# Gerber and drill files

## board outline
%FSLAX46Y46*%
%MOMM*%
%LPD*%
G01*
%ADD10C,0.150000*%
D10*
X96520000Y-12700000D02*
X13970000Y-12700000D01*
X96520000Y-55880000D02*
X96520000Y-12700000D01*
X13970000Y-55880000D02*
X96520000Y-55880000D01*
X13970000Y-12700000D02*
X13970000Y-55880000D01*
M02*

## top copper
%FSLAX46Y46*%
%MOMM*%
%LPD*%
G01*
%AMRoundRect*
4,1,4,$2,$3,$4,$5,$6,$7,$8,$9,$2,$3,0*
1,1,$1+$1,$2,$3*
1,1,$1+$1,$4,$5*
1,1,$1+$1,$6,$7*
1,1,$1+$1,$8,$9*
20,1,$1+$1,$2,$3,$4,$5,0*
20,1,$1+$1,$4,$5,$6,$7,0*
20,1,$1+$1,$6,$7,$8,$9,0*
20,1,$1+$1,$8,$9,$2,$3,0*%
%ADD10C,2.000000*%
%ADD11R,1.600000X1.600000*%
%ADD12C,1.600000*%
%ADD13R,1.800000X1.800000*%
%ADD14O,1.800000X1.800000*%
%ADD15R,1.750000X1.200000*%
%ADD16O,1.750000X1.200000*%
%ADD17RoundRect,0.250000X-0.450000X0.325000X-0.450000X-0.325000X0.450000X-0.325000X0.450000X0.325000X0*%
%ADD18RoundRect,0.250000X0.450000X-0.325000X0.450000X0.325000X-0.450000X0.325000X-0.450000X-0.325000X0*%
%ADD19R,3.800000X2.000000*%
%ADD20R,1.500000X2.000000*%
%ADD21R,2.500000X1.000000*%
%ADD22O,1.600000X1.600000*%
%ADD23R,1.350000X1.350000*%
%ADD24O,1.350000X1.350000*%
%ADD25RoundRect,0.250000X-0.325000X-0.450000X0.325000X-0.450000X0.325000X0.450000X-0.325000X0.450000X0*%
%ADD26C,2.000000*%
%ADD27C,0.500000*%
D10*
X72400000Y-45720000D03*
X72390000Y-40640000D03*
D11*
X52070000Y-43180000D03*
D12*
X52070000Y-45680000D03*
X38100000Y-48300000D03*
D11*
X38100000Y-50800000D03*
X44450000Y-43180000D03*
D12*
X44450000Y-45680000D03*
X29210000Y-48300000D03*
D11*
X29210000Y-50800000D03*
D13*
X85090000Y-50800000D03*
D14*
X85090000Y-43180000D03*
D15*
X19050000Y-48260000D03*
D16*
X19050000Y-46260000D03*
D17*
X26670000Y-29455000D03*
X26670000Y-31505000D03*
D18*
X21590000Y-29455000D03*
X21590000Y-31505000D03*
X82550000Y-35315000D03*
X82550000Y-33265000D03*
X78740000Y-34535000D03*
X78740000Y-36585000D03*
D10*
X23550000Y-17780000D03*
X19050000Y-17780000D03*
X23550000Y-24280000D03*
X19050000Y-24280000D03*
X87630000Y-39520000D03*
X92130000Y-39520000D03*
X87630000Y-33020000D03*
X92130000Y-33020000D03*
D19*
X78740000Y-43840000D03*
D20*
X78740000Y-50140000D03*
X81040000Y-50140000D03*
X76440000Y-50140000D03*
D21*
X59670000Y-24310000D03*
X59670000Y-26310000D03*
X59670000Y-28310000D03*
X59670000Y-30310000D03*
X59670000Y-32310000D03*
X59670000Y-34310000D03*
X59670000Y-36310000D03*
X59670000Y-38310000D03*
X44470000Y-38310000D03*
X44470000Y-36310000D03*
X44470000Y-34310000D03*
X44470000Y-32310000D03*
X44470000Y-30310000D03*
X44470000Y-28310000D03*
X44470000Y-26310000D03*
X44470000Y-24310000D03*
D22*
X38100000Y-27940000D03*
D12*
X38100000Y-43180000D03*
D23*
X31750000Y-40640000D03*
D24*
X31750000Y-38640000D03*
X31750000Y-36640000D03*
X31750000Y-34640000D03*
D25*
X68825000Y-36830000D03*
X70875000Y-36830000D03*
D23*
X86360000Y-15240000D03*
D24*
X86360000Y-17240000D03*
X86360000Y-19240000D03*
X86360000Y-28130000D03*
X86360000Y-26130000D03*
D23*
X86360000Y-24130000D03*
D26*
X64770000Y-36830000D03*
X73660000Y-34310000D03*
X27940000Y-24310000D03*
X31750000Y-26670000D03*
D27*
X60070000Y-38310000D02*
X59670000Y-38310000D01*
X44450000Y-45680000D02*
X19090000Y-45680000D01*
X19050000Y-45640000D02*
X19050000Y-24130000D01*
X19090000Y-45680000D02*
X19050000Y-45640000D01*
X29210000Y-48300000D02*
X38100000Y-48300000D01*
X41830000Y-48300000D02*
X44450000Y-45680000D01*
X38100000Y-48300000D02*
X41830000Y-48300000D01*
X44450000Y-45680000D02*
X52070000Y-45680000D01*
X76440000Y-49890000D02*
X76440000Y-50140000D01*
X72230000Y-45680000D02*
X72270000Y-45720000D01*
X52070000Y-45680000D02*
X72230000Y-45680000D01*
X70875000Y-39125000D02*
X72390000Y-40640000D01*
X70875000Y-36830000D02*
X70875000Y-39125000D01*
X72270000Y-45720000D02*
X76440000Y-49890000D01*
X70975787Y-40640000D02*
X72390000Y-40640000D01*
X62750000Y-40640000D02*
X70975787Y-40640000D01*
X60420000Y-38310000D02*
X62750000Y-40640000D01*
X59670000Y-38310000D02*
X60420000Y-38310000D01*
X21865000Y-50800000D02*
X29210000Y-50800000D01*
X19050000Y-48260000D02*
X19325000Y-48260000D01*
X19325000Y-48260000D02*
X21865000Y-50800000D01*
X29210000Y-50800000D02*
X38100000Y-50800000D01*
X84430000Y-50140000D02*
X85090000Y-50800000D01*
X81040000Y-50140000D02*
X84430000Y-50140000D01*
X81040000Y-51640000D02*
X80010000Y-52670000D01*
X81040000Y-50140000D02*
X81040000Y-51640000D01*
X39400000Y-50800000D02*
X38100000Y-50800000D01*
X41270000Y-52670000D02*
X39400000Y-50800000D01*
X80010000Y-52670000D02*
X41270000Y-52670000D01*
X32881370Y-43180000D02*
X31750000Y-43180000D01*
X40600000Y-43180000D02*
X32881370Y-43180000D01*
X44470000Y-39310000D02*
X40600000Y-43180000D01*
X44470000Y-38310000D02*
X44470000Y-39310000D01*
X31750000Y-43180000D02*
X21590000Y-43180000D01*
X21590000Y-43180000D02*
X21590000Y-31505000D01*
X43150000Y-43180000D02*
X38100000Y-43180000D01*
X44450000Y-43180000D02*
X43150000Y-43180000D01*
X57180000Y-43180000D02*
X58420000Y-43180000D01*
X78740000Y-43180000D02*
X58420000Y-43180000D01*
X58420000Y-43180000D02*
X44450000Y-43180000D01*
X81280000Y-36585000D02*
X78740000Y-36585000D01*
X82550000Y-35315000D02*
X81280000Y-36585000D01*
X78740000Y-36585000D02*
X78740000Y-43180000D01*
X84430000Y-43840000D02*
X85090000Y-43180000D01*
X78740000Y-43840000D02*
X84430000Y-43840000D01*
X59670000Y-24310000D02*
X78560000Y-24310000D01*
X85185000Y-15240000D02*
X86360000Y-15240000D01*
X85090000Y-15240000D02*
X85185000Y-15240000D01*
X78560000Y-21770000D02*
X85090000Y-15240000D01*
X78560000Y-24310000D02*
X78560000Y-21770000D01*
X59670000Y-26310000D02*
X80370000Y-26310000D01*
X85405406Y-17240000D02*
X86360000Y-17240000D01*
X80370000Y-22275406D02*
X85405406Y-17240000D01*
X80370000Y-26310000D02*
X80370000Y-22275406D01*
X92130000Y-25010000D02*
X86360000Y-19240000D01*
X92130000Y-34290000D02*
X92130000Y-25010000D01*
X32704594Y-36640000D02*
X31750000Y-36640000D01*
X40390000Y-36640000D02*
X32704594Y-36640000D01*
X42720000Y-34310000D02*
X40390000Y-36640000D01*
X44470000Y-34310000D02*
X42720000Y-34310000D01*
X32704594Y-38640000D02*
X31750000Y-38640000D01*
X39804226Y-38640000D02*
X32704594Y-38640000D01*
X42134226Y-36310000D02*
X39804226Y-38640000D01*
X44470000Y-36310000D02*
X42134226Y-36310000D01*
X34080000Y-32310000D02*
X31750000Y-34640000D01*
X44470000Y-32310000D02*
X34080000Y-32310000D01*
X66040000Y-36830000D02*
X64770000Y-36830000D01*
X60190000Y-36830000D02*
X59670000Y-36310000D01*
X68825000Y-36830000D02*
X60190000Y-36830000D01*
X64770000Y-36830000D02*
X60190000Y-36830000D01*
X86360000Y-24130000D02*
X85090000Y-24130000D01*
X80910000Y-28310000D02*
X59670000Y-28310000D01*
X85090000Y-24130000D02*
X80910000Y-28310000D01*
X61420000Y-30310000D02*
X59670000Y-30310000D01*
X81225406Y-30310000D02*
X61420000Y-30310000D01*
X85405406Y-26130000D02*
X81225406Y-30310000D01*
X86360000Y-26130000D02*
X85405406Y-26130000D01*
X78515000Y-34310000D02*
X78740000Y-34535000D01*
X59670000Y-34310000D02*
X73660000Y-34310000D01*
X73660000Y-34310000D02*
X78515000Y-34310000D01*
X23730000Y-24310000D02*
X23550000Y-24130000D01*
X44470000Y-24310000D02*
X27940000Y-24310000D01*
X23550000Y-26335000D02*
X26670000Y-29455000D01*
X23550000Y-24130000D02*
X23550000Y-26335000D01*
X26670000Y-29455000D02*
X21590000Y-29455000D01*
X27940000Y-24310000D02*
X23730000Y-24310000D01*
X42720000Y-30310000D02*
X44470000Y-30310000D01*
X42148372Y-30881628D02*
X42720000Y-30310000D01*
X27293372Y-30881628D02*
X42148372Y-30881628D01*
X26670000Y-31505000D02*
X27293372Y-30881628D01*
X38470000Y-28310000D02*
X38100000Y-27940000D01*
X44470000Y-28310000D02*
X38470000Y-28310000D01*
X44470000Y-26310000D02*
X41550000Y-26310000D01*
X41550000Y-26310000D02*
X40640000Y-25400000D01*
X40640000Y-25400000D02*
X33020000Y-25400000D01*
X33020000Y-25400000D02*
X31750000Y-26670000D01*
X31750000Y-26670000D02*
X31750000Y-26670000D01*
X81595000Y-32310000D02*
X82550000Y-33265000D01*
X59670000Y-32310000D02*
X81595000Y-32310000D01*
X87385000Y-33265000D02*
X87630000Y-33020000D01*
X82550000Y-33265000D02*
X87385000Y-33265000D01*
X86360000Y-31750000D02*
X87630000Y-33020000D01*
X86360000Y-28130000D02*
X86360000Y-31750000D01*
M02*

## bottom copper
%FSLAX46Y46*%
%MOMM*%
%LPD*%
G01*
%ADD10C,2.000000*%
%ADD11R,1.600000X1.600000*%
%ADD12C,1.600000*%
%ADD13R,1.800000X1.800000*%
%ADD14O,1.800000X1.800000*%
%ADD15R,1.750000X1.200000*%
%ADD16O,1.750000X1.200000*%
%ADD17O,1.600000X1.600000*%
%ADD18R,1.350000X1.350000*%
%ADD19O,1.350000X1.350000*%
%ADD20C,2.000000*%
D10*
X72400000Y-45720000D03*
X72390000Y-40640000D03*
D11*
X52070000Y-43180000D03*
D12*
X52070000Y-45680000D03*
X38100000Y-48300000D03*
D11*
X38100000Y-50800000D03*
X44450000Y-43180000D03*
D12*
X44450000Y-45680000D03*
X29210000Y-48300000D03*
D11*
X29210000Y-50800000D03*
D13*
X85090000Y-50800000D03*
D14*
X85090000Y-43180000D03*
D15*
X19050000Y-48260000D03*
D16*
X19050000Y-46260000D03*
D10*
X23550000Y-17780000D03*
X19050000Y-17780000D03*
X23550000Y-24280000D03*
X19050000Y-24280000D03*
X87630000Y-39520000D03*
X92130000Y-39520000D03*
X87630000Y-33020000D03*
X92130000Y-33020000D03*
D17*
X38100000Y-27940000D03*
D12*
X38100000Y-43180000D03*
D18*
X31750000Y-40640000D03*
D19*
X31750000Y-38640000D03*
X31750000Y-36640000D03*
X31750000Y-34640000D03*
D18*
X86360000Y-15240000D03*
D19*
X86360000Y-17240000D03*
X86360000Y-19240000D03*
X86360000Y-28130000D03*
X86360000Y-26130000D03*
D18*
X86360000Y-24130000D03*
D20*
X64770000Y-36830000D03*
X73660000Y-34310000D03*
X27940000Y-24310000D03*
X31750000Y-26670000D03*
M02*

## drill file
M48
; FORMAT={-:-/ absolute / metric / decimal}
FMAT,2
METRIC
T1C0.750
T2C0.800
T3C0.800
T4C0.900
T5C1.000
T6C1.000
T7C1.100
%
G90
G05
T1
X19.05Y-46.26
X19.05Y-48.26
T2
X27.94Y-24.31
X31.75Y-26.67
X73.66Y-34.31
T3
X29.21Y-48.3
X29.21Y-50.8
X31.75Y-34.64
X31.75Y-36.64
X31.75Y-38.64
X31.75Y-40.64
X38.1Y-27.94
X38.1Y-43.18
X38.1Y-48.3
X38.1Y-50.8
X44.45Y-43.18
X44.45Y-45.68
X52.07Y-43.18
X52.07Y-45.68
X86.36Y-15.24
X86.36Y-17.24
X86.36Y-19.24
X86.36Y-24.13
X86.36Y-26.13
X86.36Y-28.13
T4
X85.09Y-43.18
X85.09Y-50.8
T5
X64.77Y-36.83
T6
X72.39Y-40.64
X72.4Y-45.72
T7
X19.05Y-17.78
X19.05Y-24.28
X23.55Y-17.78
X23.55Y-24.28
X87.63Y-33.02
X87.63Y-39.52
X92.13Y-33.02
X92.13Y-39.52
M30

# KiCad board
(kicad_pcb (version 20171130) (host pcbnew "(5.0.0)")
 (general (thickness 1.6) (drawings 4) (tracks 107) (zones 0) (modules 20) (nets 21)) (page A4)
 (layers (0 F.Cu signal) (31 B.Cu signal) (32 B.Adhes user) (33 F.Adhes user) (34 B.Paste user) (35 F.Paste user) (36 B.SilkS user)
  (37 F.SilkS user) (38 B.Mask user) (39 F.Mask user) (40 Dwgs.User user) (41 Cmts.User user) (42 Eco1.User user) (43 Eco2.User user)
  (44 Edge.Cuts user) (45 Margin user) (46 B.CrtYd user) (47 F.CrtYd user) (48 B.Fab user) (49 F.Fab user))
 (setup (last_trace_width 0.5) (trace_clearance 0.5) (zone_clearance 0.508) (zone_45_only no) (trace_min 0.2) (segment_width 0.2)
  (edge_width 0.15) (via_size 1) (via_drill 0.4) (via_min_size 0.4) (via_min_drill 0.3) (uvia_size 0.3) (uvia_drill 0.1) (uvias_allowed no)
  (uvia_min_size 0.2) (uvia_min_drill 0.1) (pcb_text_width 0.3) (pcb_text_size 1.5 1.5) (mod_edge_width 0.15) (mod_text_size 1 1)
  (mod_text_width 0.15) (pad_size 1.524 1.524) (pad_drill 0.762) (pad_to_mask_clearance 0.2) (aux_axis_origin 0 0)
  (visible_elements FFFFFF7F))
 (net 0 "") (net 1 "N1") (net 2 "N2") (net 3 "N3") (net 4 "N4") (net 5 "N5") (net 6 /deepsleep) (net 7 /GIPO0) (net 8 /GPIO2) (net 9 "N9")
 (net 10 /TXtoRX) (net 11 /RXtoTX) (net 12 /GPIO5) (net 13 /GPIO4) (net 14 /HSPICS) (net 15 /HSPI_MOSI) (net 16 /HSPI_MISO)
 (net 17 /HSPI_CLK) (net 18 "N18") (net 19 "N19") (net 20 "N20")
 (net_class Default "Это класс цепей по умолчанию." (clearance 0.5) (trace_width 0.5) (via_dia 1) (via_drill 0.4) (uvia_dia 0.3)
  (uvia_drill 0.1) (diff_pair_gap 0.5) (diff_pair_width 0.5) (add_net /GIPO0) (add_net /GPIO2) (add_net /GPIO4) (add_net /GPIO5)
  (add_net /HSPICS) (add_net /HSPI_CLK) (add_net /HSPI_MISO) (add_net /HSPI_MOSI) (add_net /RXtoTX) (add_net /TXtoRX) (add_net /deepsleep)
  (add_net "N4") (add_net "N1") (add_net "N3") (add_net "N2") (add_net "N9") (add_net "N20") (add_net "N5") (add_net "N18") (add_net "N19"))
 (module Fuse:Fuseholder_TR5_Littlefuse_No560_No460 (layer B.Cu) (at 72.39 40.64 270)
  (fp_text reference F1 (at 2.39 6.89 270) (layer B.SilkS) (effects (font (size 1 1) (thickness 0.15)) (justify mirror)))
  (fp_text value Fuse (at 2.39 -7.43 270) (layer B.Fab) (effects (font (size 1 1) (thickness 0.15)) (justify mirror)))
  (pad 2 thru_hole circle (at 5.08 -0.01 270) (size 2 2) (drill 1) (layers *.Cu *.Mask) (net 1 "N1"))
  (pad 1 thru_hole circle (at 0 0 270) (size 2 2) (drill 1) (layers *.Cu *.Mask) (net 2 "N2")))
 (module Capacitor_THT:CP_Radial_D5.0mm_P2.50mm (layer B.Cu) (at 52.07 43.18 270)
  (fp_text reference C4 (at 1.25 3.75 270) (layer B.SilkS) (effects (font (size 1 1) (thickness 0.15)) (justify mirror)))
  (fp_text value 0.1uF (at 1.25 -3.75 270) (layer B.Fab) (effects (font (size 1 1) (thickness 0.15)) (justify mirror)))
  (pad 1 thru_hole rect (at 0 0 270) (size 1.6 1.6) (drill 0.8) (layers *.Cu *.Mask) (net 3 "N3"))
  (pad 2 thru_hole circle (at 2.5 0 270) (size 1.6 1.6) (drill 0.8) (layers *.Cu *.Mask) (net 1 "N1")))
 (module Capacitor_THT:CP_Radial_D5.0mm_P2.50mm (layer B.Cu) (at 38.1 50.8 90)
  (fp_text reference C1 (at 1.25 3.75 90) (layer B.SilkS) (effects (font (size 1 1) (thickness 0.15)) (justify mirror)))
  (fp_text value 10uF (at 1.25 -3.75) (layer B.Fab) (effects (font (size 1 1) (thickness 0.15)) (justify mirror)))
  (pad 2 thru_hole circle (at 2.5 0 90) (size 1.6 1.6) (drill 0.8) (layers *.Cu *.Mask) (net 1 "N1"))
  (pad 1 thru_hole rect (at 0 0 90) (size 1.6 1.6) (drill 0.8) (layers *.Cu *.Mask) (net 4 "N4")))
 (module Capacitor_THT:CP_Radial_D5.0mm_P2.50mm (layer B.Cu) (at 44.45 43.18 270)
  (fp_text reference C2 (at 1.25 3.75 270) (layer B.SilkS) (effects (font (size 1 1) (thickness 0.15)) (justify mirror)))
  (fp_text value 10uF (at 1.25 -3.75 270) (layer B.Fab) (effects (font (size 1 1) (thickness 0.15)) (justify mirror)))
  (pad 1 thru_hole rect (at 0 0 270) (size 1.6 1.6) (drill 0.8) (layers *.Cu *.Mask) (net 3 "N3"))
  (pad 2 thru_hole circle (at 2.5 0 270) (size 1.6 1.6) (drill 0.8) (layers *.Cu *.Mask) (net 1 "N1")))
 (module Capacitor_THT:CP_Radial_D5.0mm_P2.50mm (layer B.Cu) (at 29.21 50.8 90)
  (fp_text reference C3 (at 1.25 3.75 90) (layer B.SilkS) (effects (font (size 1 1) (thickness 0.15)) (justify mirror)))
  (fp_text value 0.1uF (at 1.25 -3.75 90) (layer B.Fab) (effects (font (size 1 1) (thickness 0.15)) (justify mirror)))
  (pad 2 thru_hole circle (at 2.5 0 90) (size 1.6 1.6) (drill 0.8) (layers *.Cu *.Mask) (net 1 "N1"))
  (pad 1 thru_hole rect (at 0 0 90) (size 1.6 1.6) (drill 0.8) (layers *.Cu *.Mask) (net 4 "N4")))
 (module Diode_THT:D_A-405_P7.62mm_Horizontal (layer B.Cu) (at 85.09 50.8 90)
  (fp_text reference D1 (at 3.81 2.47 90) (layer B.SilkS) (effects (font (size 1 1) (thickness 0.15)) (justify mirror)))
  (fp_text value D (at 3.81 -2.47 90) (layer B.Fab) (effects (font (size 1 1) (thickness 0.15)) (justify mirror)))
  (pad 1 thru_hole rect (at 0 0 90) (size 1.8 1.8) (drill 0.9) (layers *.Cu *.Mask) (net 4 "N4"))
  (pad 2 thru_hole oval (at 7.62 0 90) (size 1.8 1.8) (drill 0.9) (layers *.Cu *.Mask) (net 3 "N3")))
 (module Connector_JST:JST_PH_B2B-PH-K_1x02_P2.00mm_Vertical (layer B.Cu) (at 19.05 48.26 90)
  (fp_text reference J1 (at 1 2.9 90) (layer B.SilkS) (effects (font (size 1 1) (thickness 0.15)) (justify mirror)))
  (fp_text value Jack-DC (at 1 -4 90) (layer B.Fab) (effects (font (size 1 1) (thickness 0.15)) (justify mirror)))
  (pad 1 thru_hole rect (at 0 0 90) (size 1.2 1.75) (drill 0.75) (layers *.Cu *.Mask) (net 4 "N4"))
  (pad 2 thru_hole oval (at 2 0 90) (size 1.2 1.75) (drill 0.75) (layers *.Cu *.Mask) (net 1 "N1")))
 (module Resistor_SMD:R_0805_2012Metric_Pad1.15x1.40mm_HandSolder (layer F.Cu) (at 26.67 30.48 270)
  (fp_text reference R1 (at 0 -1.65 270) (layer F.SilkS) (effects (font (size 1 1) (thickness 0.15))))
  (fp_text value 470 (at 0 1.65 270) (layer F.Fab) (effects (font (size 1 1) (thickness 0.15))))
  (pad 1 smd roundrect (at -1.025 0 270) (size 1.15 1.4) (layers F.Cu F.Paste F.Mask) (roundrect_rratio 0.217391) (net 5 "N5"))
  (pad 2 smd roundrect (at 1.025 0 270) (size 1.15 1.4) (layers F.Cu F.Paste F.Mask) (roundrect_rratio 0.217391) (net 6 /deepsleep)))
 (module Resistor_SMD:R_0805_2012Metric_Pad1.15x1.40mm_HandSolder (layer F.Cu) (at 21.59 30.48 90)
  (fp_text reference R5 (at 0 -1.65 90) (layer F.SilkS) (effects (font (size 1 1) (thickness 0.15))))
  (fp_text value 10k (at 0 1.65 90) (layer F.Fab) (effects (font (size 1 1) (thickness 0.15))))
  (pad 2 smd roundrect (at 1.025 0 90) (size 1.15 1.4) (layers F.Cu F.Paste F.Mask) (roundrect_rratio 0.217391) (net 5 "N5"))
  (pad 1 smd roundrect (at -1.025 0 90) (size 1.15 1.4) (layers F.Cu F.Paste F.Mask) (roundrect_rratio 0.217391) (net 3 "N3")))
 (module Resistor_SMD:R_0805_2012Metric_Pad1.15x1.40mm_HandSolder (layer F.Cu) (at 82.55 34.29 90)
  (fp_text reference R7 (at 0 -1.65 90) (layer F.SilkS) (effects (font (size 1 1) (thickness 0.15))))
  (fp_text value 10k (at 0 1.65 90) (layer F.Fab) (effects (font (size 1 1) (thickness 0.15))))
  (pad 1 smd roundrect (at -1.025 0 90) (size 1.15 1.4) (layers F.Cu F.Paste F.Mask) (roundrect_rratio 0.217391) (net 3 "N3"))
  (pad 2 smd roundrect (at 1.025 0 90) (size 1.15 1.4) (layers F.Cu F.Paste F.Mask) (roundrect_rratio 0.217391) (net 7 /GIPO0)))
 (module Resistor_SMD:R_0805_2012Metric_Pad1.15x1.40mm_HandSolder (layer F.Cu) (at 78.74 35.56 90)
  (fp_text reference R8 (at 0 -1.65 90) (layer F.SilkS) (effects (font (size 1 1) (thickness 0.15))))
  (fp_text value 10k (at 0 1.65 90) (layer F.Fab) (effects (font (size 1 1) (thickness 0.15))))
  (pad 2 smd roundrect (at 1.025 0 90) (size 1.15 1.4) (layers F.Cu F.Paste F.Mask) (roundrect_rratio 0.217391) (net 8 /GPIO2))
  (pad 1 smd roundrect (at -1.025 0 90) (size 1.15 1.4) (layers F.Cu F.Paste F.Mask) (roundrect_rratio 0.217391) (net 3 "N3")))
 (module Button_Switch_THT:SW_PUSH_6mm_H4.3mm (layer B.Cu) (at 19.05 17.78 270)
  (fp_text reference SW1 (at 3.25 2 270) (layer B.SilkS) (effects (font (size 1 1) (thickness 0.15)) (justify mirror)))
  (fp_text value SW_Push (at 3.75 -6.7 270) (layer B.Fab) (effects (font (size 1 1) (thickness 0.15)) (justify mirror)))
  (pad 2 thru_hole circle (at 0 -4.5 180) (size 2 2) (drill 1.1) (layers *.Cu *.Mask) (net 5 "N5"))
  (pad 1 thru_hole circle (at 0 0 180) (size 2 2) (drill 1.1) (layers *.Cu *.Mask) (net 1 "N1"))
  (pad 2 thru_hole circle (at 6.5 -4.5 180) (size 2 2) (drill 1.1) (layers *.Cu *.Mask) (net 5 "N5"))
  (pad 1 thru_hole circle (at 6.5 0 180) (size 2 2) (drill 1.1) (layers *.Cu *.Mask) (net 1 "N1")))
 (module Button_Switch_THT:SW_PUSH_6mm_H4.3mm (layer B.Cu) (at 87.63 33.02 270)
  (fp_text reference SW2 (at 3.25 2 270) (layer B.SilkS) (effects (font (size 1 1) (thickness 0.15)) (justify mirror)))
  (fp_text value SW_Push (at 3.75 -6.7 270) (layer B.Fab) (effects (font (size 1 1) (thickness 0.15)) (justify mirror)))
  (pad 1 thru_hole circle (at 6.5 0 180) (size 2 2) (drill 1.1) (layers *.Cu *.Mask) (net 7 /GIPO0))
  (pad 2 thru_hole circle (at 6.5 -4.5 180) (size 2 2) (drill 1.1) (layers *.Cu *.Mask) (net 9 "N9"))
  (pad 1 thru_hole circle (at 0 0 180) (size 2 2) (drill 1.1) (layers *.Cu *.Mask) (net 7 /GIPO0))
  (pad 2 thru_hole circle (at 0 -4.5 180) (size 2 2) (drill 1.1) (layers *.Cu *.Mask) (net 9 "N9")))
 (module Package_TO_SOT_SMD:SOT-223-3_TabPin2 (layer F.Cu) (at 78.74 46.99 90)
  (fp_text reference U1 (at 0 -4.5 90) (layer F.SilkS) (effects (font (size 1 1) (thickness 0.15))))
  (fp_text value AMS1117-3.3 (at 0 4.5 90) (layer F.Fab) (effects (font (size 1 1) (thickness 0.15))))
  (pad 2 smd rect (at 3.15 0 90) (size 2 3.8) (layers F.Cu F.Paste F.Mask) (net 3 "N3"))
  (pad 2 smd rect (at -3.15 0 90) (size 2 1.5) (layers F.Cu F.Paste F.Mask) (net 3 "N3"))
  (pad 3 smd rect (at -3.15 2.3 90) (size 2 1.5) (layers F.Cu F.Paste F.Mask) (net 4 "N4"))
  (pad 1 smd rect (at -3.15 -2.3 90) (size 2 1.5) (layers F.Cu F.Paste F.Mask) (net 1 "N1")))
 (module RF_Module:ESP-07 (layer F.Cu) (at 52.07 29.21)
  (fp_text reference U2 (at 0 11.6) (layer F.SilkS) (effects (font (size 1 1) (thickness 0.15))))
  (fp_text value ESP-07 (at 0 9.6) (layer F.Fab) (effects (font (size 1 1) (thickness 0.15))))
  (pad 16 smd rect (at 7.6 -4.9) (size 2.5 1) (layers F.Cu F.Paste F.Mask) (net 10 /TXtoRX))
  (pad 15 smd rect (at 7.6 -2.9) (size 2.5 1) (layers F.Cu F.Paste F.Mask) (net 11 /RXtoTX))
  (pad 14 smd rect (at 7.6 -0.9) (size 2.5 1) (layers F.Cu F.Paste F.Mask) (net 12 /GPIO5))
  (pad 13 smd rect (at 7.6 1.1) (size 2.5 1) (layers F.Cu F.Paste F.Mask) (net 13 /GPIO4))
  (pad 12 smd rect (at 7.6 3.1) (size 2.5 1) (layers F.Cu F.Paste F.Mask) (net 7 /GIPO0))
  (pad 11 smd rect (at 7.6 5.1) (size 2.5 1) (layers F.Cu F.Paste F.Mask) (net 8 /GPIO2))
  (pad 10 smd rect (at 7.6 7.1) (size 2.5 1) (layers F.Cu F.Paste F.Mask) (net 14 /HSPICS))
  (pad 9 smd rect (at 7.6 9.1) (size 2.5 1) (layers F.Cu F.Paste F.Mask) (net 2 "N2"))
  (pad 8 smd rect (at -7.6 9.1) (size 2.5 1) (layers F.Cu F.Paste F.Mask) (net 3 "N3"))
  (pad 7 smd rect (at -7.6 7.1) (size 2.5 1) (layers F.Cu F.Paste F.Mask) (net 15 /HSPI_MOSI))
  (pad 6 smd rect (at -7.6 5.1) (size 2.5 1) (layers F.Cu F.Paste F.Mask) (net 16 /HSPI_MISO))
  (pad 5 smd rect (at -7.6 3.1) (size 2.5 1) (layers F.Cu F.Paste F.Mask) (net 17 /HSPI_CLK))
  (pad 4 smd rect (at -7.6 1.1) (size 2.5 1) (layers F.Cu F.Paste F.Mask) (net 6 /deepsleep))
  (pad 3 smd rect (at -7.6 -0.9) (size 2.5 1) (layers F.Cu F.Paste F.Mask) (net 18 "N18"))
  (pad 2 smd rect (at -7.6 -2.9) (size 2.5 1) (layers F.Cu F.Paste F.Mask) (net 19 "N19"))
  (pad 1 smd rect (at -7.6 -4.9) (size 2.5 1) (layers F.Cu F.Paste F.Mask) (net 5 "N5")))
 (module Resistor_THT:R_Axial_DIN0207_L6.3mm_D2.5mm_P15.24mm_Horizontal (layer B.Cu) (at 38.1 43.18 90)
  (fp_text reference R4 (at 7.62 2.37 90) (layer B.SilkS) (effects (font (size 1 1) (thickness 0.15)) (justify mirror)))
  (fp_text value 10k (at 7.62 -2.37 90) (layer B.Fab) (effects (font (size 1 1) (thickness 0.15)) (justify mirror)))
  (pad 2 thru_hole oval (at 15.24 0 90) (size 1.6 1.6) (drill 0.8) (layers *.Cu *.Mask) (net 18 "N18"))
  (pad 1 thru_hole circle (at 0 0 90) (size 1.6 1.6) (drill 0.8) (layers *.Cu *.Mask) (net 3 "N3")))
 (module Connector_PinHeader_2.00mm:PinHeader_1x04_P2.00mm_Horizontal (layer F.Cu) (at 31.75 40.64 180)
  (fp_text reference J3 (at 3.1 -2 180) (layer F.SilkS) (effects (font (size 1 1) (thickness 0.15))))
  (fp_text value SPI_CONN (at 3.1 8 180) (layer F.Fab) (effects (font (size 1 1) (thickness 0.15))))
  (pad 1 thru_hole rect (at 0 0 180) (size 1.35 1.35) (drill 0.8) (layers *.Cu *.Mask) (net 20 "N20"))
  (pad 2 thru_hole oval (at 0 2 180) (size 1.35 1.35) (drill 0.8) (layers *.Cu *.Mask) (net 15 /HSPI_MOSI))
  (pad 3 thru_hole oval (at 0 4 180) (size 1.35 1.35) (drill 0.8) (layers *.Cu *.Mask) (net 16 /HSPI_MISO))
  (pad 4 thru_hole oval (at 0 6 180) (size 1.35 1.35) (drill 0.8) (layers *.Cu *.Mask) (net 17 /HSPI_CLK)))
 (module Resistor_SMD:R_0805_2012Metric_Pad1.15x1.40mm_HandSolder (layer F.Cu) (at 69.85 36.83)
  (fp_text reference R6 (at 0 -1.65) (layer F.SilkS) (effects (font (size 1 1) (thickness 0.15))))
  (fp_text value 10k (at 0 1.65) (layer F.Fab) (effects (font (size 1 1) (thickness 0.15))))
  (pad 1 smd roundrect (at -1.025 0) (size 1.15 1.4) (layers F.Cu F.Paste F.Mask) (roundrect_rratio 0.217391) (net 14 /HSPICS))
  (pad 2 smd roundrect (at 1.025 0) (size 1.15 1.4) (layers F.Cu F.Paste F.Mask) (roundrect_rratio 0.217391) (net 2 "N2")))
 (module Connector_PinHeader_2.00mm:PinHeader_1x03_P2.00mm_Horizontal (layer F.Cu) (at 86.36 15.24)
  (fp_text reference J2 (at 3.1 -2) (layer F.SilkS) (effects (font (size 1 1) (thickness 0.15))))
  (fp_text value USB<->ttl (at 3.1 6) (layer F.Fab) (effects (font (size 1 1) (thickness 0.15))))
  (pad 1 thru_hole rect (at 0 0) (size 1.35 1.35) (drill 0.8) (layers *.Cu *.Mask) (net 10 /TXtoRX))
  (pad 2 thru_hole oval (at 0 2) (size 1.35 1.35) (drill 0.8) (layers *.Cu *.Mask) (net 11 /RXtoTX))
  (pad 3 thru_hole oval (at 0 4) (size 1.35 1.35) (drill 0.8) (layers *.Cu *.Mask) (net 9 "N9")))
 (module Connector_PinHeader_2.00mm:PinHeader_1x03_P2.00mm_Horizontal (layer F.Cu) (at 86.36 24.13)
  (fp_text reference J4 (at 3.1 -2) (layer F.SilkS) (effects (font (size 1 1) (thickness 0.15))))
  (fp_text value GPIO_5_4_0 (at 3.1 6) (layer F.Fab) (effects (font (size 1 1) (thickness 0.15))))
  (pad 3 thru_hole oval (at 0 4) (size 1.35 1.35) (drill 0.8) (layers *.Cu *.Mask) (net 7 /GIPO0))
  (pad 2 thru_hole oval (at 0 2) (size 1.35 1.35) (drill 0.8) (layers *.Cu *.Mask) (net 13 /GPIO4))
  (pad 1 thru_hole rect (at 0 0) (size 1.35 1.35) (drill 0.8) (layers *.Cu *.Mask) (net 12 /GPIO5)))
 (gr_line (start 96.52 12.7) (end 13.97 12.7) (layer Edge.Cuts) (width 0.15))
 (gr_line (start 96.52 55.88) (end 96.52 12.7) (layer Edge.Cuts) (width 0.15))
 (gr_line (start 13.97 55.88) (end 96.52 55.88) (layer Edge.Cuts) (width 0.15))
 (gr_line (start 13.97 12.7) (end 13.97 55.88) (layer Edge.Cuts) (width 0.15))
 (segment (start 60.07 38.31) (end 59.67 38.31) (width 0.5) (layer F.Cu) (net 2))
 (segment (start 44.45 45.68) (end 19.09 45.68) (width 0.5) (layer F.Cu) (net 1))
 (segment (start 19.05 45.64) (end 19.05 24.13) (width 0.5) (layer F.Cu) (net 1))
 (segment (start 19.09 45.68) (end 19.05 45.64) (width 0.5) (layer F.Cu) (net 1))
 (segment (start 29.21 48.3) (end 38.1 48.3) (width 0.5) (layer F.Cu) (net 1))
 (segment (start 41.83 48.3) (end 44.45 45.68) (width 0.5) (layer F.Cu) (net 1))
 (segment (start 38.1 48.3) (end 41.83 48.3) (width 0.5) (layer F.Cu) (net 1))
 (segment (start 44.45 45.68) (end 52.07 45.68) (width 0.5) (layer F.Cu) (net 1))
 (segment (start 76.44 49.89) (end 76.44 50.14) (width 0.5) (layer F.Cu) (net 1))
 (segment (start 72.23 45.68) (end 72.27 45.72) (width 0.5) (layer F.Cu) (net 1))
 (segment (start 52.07 45.68) (end 72.23 45.68) (width 0.5) (layer F.Cu) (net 1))
 (segment (start 70.875 39.125) (end 72.39 40.64) (width 0.5) (layer F.Cu) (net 2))
 (segment (start 70.875 36.83) (end 70.875 39.125) (width 0.5) (layer F.Cu) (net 2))
 (segment (start 72.27 45.72) (end 76.44 49.89) (width 0.5) (layer F.Cu) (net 1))
 (segment (start 70.975787 40.64) (end 72.39 40.64) (width 0.5) (layer F.Cu) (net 2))
 (segment (start 62.75 40.64) (end 70.975787 40.64) (width 0.5) (layer F.Cu) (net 2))
 (segment (start 60.42 38.31) (end 62.75 40.64) (width 0.5) (layer F.Cu) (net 2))
 (segment (start 59.67 38.31) (end 60.42 38.31) (width 0.5) (layer F.Cu) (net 2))
 (segment (start 21.865 50.8) (end 29.21 50.8) (width 0.5) (layer F.Cu) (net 4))
 (segment (start 19.05 48.26) (end 19.325 48.26) (width 0.5) (layer F.Cu) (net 4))
 (segment (start 19.325 48.26) (end 21.865 50.8) (width 0.5) (layer F.Cu) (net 4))
 (segment (start 29.21 50.8) (end 38.1 50.8) (width 0.5) (layer F.Cu) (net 4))
 (segment (start 84.43 50.14) (end 85.09 50.8) (width 0.5) (layer F.Cu) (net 4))
 (segment (start 81.04 50.14) (end 84.43 50.14) (width 0.5) (layer F.Cu) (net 4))
 (segment (start 81.04 51.64) (end 80.01 52.67) (width 0.5) (layer F.Cu) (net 4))
 (segment (start 81.04 50.14) (end 81.04 51.64) (width 0.5) (layer F.Cu) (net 4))
 (segment (start 39.4 50.8) (end 38.1 50.8) (width 0.5) (layer F.Cu) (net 4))
 (segment (start 41.27 52.67) (end 39.4 50.8) (width 0.5) (layer F.Cu) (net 4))
 (segment (start 80.01 52.67) (end 41.27 52.67) (width 0.5) (layer F.Cu) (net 4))
 (segment (start 32.88137 43.18) (end 31.75 43.18) (width 0.5) (layer F.Cu) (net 3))
 (segment (start 40.6 43.18) (end 32.88137 43.18) (width 0.5) (layer F.Cu) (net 3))
 (segment (start 44.47 39.31) (end 40.6 43.18) (width 0.5) (layer F.Cu) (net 3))
 (segment (start 44.47 38.31) (end 44.47 39.31) (width 0.5) (layer F.Cu) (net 3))
 (segment (start 31.75 43.18) (end 21.59 43.18) (width 0.5) (layer F.Cu) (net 3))
 (segment (start 21.59 43.18) (end 21.59 31.505) (width 0.5) (layer F.Cu) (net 3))
 (segment (start 43.15 43.18) (end 38.1 43.18) (width 0.5) (layer F.Cu) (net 3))
 (segment (start 44.45 43.18) (end 43.15 43.18) (width 0.5) (layer F.Cu) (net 3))
 (segment (start 57.18 43.18) (end 58.42 43.18) (width 0.5) (layer F.Cu) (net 3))
 (segment (start 78.74 43.18) (end 58.42 43.18) (width 0.5) (layer F.Cu) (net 3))
 (segment (start 58.42 43.18) (end 44.45 43.18) (width 0.5) (layer F.Cu) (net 3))
 (segment (start 81.28 36.585) (end 78.74 36.585) (width 0.5) (layer F.Cu) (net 3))
 (segment (start 82.55 35.315) (end 81.28 36.585) (width 0.5) (layer F.Cu) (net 3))
 (segment (start 78.74 36.585) (end 78.74 43.18) (width 0.5) (layer F.Cu) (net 3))
 (segment (start 84.43 43.84) (end 85.09 43.18) (width 0.5) (layer F.Cu) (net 3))
 (segment (start 78.74 43.84) (end 84.43 43.84) (width 0.5) (layer F.Cu) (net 3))
 (segment (start 59.67 24.31) (end 78.56 24.31) (width 0.5) (layer F.Cu) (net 10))
 (segment (start 85.185 15.24) (end 86.36 15.24) (width 0.5) (layer F.Cu) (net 10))
 (segment (start 85.09 15.24) (end 85.185 15.24) (width 0.5) (layer F.Cu) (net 10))
 (segment (start 78.56 21.77) (end 85.09 15.24) (width 0.5) (layer F.Cu) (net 10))
 (segment (start 78.56 24.31) (end 78.56 21.77) (width 0.5) (layer F.Cu) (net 10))
 (segment (start 59.67 26.31) (end 80.37 26.31) (width 0.5) (layer F.Cu) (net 11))
 (segment (start 85.405406 17.24) (end 86.36 17.24) (width 0.5) (layer F.Cu) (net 11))
 (segment (start 80.37 22.275406) (end 85.405406 17.24) (width 0.5) (layer F.Cu) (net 11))
 (segment (start 80.37 26.31) (end 80.37 22.275406) (width 0.5) (layer F.Cu) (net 11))
 (segment (start 92.13 25.01) (end 86.36 19.24) (width 0.5) (layer F.Cu) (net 9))
 (segment (start 92.13 34.29) (end 92.13 25.01) (width 0.5) (layer F.Cu) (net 9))
 (segment (start 32.704594 36.64) (end 31.75 36.64) (width 0.5) (layer F.Cu) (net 16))
 (segment (start 40.39 36.64) (end 32.704594 36.64) (width 0.5) (layer F.Cu) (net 16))
 (segment (start 42.72 34.31) (end 40.39 36.64) (width 0.5) (layer F.Cu) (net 16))
 (segment (start 44.47 34.31) (end 42.72 34.31) (width 0.5) (layer F.Cu) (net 16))
 (segment (start 32.704594 38.64) (end 31.75 38.64) (width 0.5) (layer F.Cu) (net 15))
 (segment (start 39.804226 38.64) (end 32.704594 38.64) (width 0.5) (layer F.Cu) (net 15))
 (segment (start 42.134226 36.31) (end 39.804226 38.64) (width 0.5) (layer F.Cu) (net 15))
 (segment (start 44.47 36.31) (end 42.134226 36.31) (width 0.5) (layer F.Cu) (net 15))
 (segment (start 34.08 32.31) (end 31.75 34.64) (width 0.5) (layer F.Cu) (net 17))
 (segment (start 44.47 32.31) (end 34.08 32.31) (width 0.5) (layer F.Cu) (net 17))
 (segment (start 66.04 36.83) (end 64.77 36.83) (width 0.5) (layer F.Cu) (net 14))
 (segment (start 60.19 36.83) (end 59.67 36.31) (width 0.5) (layer F.Cu) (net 14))
 (segment (start 68.825 36.83) (end 60.19 36.83) (width 0.5) (layer F.Cu) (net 14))
 (segment (start 64.77 36.83) (end 60.19 36.83) (width 0.5) (layer F.Cu) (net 14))
 (via (at 64.77 36.83) (size 2) (drill 1) (layers F.Cu B.Cu) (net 14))
 (segment (start 86.36 24.13) (end 85.09 24.13) (width 0.5) (layer F.Cu) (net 12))
 (segment (start 80.91 28.31) (end 59.67 28.31) (width 0.5) (layer F.Cu) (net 12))
 (segment (start 85.09 24.13) (end 80.91 28.31) (width 0.5) (layer F.Cu) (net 12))
 (segment (start 61.42 30.31) (end 59.67 30.31) (width 0.5) (layer F.Cu) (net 13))
 (segment (start 81.225406 30.31) (end 61.42 30.31) (width 0.5) (layer F.Cu) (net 13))
 (segment (start 85.405406 26.13) (end 81.225406 30.31) (width 0.5) (layer F.Cu) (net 13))
 (segment (start 86.36 26.13) (end 85.405406 26.13) (width 0.5) (layer F.Cu) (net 13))
 (segment (start 78.515 34.31) (end 78.74 34.535) (width 0.5) (layer F.Cu) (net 8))
 (segment (start 59.67 34.31) (end 73.66 34.31) (width 0.5) (layer F.Cu) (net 8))
 (segment (start 73.66 34.31) (end 78.515 34.31) (width 0.5) (layer F.Cu) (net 8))
 (via (at 73.66 34.31) (size 2) (drill 0.8) (layers F.Cu B.Cu) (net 8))
 (segment (start 23.73 24.31) (end 23.55 24.13) (width 0.5) (layer F.Cu) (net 5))
 (segment (start 44.47 24.31) (end 27.94 24.31) (width 0.5) (layer F.Cu) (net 5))
 (segment (start 23.55 26.335) (end 26.67 29.455) (width 0.5) (layer F.Cu) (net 5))
 (segment (start 23.55 24.13) (end 23.55 26.335) (width 0.5) (layer F.Cu) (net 5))
 (segment (start 26.67 29.455) (end 21.59 29.455) (width 0.5) (layer F.Cu) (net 5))
 (segment (start 27.94 24.31) (end 23.73 24.31) (width 0.5) (layer F.Cu) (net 5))
 (via (at 27.94 24.31) (size 2) (drill 0.8) (layers F.Cu B.Cu) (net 5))
 (segment (start 42.72 30.31) (end 44.47 30.31) (width 0.5) (layer F.Cu) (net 6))
 (segment (start 42.148372 30.881628) (end 42.72 30.31) (width 0.5) (layer F.Cu) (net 6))
 (segment (start 27.293372 30.881628) (end 42.148372 30.881628) (width 0.5) (layer F.Cu) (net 6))
 (segment (start 26.67 31.505) (end 27.293372 30.881628) (width 0.5) (layer F.Cu) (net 6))
 (segment (start 38.47 28.31) (end 38.1 27.94) (width 0.5) (layer F.Cu) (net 18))
 (segment (start 44.47 28.31) (end 38.47 28.31) (width 0.5) (layer F.Cu) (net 18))
 (segment (start 44.47 26.31) (end 41.55 26.31) (width 0.5) (layer F.Cu) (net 19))
 (segment (start 41.55 26.31) (end 40.64 25.4) (width 0.5) (layer F.Cu) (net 19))
 (segment (start 40.64 25.4) (end 33.02 25.4) (width 0.5) (layer F.Cu) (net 19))
 (segment (start 33.02 25.4) (end 31.75 26.67) (width 0.5) (layer F.Cu) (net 19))
 (segment (start 31.75 26.67) (end 31.75 26.67) (width 0.5) (layer F.Cu) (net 19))
 (via (at 31.75 26.67) (size 2) (drill 0.8) (layers F.Cu B.Cu) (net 19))
 (segment (start 81.595 32.31) (end 82.55 33.265) (width 0.5) (layer F.Cu) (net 7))
 (segment (start 59.67 32.31) (end 81.595 32.31) (width 0.5) (layer F.Cu) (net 7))
 (segment (start 87.385 33.265) (end 87.63 33.02) (width 0.5) (layer F.Cu) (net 7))
 (segment (start 82.55 33.265) (end 87.385 33.265) (width 0.5) (layer F.Cu) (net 7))
 (segment (start 86.36 31.75) (end 87.63 33.02) (width 0.5) (layer F.Cu) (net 7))
 (segment (start 86.36 28.13) (end 86.36 31.75) (width 0.5) (layer F.Cu) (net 7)))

